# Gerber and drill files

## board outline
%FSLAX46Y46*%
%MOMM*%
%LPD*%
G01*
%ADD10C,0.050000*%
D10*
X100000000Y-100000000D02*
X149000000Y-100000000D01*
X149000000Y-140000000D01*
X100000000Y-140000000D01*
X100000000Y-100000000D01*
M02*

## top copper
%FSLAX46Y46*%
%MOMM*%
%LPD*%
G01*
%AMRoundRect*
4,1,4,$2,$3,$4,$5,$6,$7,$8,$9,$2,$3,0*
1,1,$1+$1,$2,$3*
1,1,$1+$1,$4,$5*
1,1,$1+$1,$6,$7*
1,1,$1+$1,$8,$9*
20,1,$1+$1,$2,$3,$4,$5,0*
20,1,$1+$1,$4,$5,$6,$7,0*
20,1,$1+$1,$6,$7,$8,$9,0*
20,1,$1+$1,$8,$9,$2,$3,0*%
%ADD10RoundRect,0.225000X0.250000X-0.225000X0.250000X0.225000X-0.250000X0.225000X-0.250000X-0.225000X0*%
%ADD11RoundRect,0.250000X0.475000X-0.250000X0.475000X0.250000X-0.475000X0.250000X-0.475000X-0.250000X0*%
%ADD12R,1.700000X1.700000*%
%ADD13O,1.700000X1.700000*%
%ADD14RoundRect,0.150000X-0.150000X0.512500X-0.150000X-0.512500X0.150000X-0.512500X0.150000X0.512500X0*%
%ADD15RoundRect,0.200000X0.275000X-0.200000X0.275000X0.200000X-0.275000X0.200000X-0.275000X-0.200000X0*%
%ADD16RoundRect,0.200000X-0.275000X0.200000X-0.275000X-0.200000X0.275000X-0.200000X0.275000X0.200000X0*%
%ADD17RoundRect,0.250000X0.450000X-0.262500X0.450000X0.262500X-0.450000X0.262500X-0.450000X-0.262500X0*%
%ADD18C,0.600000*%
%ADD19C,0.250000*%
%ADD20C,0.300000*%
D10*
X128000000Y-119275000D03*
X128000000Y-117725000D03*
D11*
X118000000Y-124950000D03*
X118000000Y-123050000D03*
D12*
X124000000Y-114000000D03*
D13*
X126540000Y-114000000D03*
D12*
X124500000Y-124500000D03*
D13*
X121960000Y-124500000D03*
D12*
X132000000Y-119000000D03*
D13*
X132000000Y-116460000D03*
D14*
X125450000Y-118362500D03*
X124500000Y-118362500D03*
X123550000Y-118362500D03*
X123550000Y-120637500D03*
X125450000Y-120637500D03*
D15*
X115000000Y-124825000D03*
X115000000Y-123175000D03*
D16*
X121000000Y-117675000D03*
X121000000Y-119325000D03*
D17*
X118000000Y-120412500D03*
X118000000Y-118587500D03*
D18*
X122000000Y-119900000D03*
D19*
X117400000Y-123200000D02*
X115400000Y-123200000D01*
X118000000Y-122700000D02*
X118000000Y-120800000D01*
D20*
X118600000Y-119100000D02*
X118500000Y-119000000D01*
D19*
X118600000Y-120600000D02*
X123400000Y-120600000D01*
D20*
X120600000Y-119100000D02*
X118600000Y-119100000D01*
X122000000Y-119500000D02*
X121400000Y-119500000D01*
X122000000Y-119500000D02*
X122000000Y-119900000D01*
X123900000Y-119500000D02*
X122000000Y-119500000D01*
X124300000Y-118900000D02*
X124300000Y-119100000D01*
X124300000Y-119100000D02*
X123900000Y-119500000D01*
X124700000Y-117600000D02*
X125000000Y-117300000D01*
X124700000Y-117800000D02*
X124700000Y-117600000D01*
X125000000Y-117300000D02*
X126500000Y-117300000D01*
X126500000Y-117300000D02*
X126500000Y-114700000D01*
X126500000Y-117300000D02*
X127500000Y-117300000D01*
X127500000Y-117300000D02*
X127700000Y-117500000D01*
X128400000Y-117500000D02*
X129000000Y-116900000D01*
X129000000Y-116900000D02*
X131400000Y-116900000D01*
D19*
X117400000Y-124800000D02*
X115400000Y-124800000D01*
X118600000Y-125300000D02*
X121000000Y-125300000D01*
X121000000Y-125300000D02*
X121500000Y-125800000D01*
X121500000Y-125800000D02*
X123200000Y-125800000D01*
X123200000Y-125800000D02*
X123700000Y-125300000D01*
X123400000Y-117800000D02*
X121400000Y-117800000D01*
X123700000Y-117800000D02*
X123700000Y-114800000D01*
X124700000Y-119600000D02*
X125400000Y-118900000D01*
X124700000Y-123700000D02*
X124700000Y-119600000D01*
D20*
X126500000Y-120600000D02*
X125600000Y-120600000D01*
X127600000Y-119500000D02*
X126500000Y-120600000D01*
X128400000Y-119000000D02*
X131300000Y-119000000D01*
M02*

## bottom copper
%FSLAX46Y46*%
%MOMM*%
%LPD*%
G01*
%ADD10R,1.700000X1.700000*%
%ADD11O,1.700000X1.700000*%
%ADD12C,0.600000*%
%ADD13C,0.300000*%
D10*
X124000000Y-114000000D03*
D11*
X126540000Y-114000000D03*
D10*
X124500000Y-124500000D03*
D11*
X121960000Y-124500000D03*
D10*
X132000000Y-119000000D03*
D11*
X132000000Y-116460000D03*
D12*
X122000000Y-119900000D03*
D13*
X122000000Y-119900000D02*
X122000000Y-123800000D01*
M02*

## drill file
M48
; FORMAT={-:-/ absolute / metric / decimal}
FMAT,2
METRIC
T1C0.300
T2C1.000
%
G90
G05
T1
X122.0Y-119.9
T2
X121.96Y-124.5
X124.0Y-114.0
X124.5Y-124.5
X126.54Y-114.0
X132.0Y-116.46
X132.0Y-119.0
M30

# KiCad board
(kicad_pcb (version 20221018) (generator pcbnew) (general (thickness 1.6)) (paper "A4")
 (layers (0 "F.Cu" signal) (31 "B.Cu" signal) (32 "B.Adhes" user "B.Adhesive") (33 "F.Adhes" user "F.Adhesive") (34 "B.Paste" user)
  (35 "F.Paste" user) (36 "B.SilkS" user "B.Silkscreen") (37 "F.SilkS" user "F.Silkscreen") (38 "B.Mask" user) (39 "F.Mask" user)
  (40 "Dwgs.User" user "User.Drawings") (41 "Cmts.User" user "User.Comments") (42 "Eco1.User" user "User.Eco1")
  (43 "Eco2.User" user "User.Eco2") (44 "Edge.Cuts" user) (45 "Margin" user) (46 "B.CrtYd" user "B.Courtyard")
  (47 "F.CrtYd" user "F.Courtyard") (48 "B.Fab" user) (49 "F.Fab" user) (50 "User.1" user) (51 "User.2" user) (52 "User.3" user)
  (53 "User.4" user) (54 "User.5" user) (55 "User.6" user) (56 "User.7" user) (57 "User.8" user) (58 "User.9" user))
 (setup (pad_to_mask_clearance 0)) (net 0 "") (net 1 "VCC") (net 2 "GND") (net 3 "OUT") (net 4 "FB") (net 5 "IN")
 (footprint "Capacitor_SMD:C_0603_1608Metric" (layer "F.Cu") (at 128 118.5 90)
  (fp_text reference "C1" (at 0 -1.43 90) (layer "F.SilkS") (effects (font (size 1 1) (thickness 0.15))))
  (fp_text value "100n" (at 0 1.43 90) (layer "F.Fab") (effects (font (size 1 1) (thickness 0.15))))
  (pad "1" smd roundrect (at -0.775 0 90) (size 0.9 0.95) (layers "F.Cu" "F.Paste" "F.Mask") (roundrect_rratio 0.25) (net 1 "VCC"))
  (pad "2" smd roundrect (at 0.775 0 90) (size 0.9 0.95) (layers "F.Cu" "F.Paste" "F.Mask") (roundrect_rratio 0.25) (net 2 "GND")))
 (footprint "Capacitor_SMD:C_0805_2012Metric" (layer "F.Cu") (at 118 124 90)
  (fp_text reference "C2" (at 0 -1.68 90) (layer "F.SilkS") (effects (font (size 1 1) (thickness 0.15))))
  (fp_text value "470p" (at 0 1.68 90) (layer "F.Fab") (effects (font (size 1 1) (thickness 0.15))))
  (pad "1" smd roundrect (at -0.95 0 90) (size 1 1.45) (layers "F.Cu" "F.Paste" "F.Mask") (roundrect_rratio 0.25) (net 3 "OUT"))
  (pad "2" smd roundrect (at 0.95 0 90) (size 1 1.45) (layers "F.Cu" "F.Paste" "F.Mask") (roundrect_rratio 0.25) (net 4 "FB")))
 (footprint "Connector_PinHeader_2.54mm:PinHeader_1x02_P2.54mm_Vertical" (layer "F.Cu") (at 124 114 90)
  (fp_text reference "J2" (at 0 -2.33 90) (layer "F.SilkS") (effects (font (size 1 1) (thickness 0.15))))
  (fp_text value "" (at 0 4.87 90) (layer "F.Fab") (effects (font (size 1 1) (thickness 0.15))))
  (pad "1" thru_hole rect (at 0 0 90) (size 1.7 1.7) (drill 1) (layers "*.Cu" "*.Mask") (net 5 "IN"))
  (pad "2" thru_hole oval (at 0 2.54 90) (size 1.7 1.7) (drill 1) (layers "*.Cu" "*.Mask") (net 2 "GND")))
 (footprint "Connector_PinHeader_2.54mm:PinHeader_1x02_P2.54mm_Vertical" (layer "F.Cu") (at 124.5 124.5 -90)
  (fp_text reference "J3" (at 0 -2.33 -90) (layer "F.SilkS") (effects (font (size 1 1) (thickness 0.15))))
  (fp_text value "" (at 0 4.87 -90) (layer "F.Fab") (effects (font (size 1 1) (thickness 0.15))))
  (pad "1" thru_hole rect (at 0 0 270) (size 1.7 1.7) (drill 1) (layers "*.Cu" "*.Mask") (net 3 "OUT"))
  (pad "2" thru_hole oval (at 0 2.54 270) (size 1.7 1.7) (drill 1) (layers "*.Cu" "*.Mask") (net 2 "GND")))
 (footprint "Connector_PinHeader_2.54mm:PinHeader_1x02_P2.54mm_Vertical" (layer "F.Cu") (at 132 119 180)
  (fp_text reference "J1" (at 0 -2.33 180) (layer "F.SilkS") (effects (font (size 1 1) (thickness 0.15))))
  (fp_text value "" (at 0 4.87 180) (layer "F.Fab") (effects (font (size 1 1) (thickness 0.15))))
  (pad "1" thru_hole rect (at 0 0 180) (size 1.7 1.7) (drill 1) (layers "*.Cu" "*.Mask") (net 1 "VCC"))
  (pad "2" thru_hole oval (at 0 2.54 180) (size 1.7 1.7) (drill 1) (layers "*.Cu" "*.Mask") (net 2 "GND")))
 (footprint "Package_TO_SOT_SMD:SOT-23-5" (layer "F.Cu") (at 124.5 119.5 -90)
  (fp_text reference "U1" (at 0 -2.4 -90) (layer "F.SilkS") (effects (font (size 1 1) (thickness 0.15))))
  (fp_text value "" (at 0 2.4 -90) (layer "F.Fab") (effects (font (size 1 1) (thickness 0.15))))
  (pad "1" smd roundrect (at -1.1375 -0.95 270) (size 1.325 0.6) (layers "F.Cu" "F.Paste" "F.Mask") (roundrect_rratio 0.25) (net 3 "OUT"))
  (pad "2" smd roundrect (at -1.1375 0 270) (size 1.325 0.6) (layers "F.Cu" "F.Paste" "F.Mask") (roundrect_rratio 0.25) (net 2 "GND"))
  (pad "3" smd roundrect (at -1.1375 0.95 270) (size 1.325 0.6) (layers "F.Cu" "F.Paste" "F.Mask") (roundrect_rratio 0.25) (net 5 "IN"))
  (pad "4" smd roundrect (at 1.1375 0.95 270) (size 1.325 0.6) (layers "F.Cu" "F.Paste" "F.Mask") (roundrect_rratio 0.25) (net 4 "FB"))
  (pad "5" smd roundrect (at 1.1375 -0.95 270) (size 1.325 0.6) (layers "F.Cu" "F.Paste" "F.Mask") (roundrect_rratio 0.25) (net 1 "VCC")))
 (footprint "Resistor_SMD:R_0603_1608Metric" (layer "F.Cu") (at 115 124 90)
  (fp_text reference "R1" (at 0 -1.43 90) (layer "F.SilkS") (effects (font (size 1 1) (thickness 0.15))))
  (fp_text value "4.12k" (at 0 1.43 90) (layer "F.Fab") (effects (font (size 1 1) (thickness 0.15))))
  (pad "1" smd roundrect (at -0.825 0 90) (size 0.8 0.95) (layers "F.Cu" "F.Paste" "F.Mask") (roundrect_rratio 0.25) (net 3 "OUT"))
  (pad "2" smd roundrect (at 0.825 0 90) (size 0.8 0.95) (layers "F.Cu" "F.Paste" "F.Mask") (roundrect_rratio 0.25) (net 4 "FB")))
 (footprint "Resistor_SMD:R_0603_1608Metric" (layer "F.Cu") (at 121 118.5 -90)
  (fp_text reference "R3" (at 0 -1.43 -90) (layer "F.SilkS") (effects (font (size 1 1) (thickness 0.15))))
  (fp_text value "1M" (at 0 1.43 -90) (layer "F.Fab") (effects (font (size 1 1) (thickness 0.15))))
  (pad "1" smd roundrect (at -0.825 0 270) (size 0.8 0.95) (layers "F.Cu" "F.Paste" "F.Mask") (roundrect_rratio 0.25) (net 5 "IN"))
  (pad "2" smd roundrect (at 0.825 0 270) (size 0.8 0.95) (layers "F.Cu" "F.Paste" "F.Mask") (roundrect_rratio 0.25) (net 2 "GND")))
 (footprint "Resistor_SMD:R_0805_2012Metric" (layer "F.Cu") (at 118 119.5 90)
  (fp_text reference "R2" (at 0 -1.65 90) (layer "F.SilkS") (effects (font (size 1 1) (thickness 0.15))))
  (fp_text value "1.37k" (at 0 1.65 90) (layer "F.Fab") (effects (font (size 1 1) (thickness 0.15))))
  (pad "1" smd roundrect (at -0.9125 0 90) (size 1.025 1.4) (layers "F.Cu" "F.Paste" "F.Mask") (roundrect_rratio 0.243902) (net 4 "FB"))
  (pad "2" smd roundrect (at 0.9125 0 90) (size 1.025 1.4) (layers "F.Cu" "F.Paste" "F.Mask") (roundrect_rratio 0.243902) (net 2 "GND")))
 (gr_rect (start 100 100) (end 149 140) (stroke (width 0.05) (type default)) (fill none) (layer "Edge.Cuts"))
 (segment (start 117.4 123.2) (end 115.4 123.2) (width 0.25) (layer "F.Cu") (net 4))
 (segment (start 118 122.7) (end 118 120.8) (width 0.25) (layer "F.Cu") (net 4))
 (segment (start 118.6 119.1) (end 118.5 119) (width 0.3) (layer "F.Cu") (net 2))
 (segment (start 118.6 120.6) (end 123.4 120.6) (width 0.25) (layer "F.Cu") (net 4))
 (segment (start 120.6 119.1) (end 118.6 119.1) (width 0.3) (layer "F.Cu") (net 2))
 (segment (start 122 119.5) (end 121.4 119.5) (width 0.3) (layer "F.Cu") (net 2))
 (segment (start 122 119.5) (end 122 119.9) (width 0.3) (layer "F.Cu") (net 2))
 (segment (start 123.9 119.5) (end 122 119.5) (width 0.3) (layer "F.Cu") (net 2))
 (segment (start 124.3 118.9) (end 124.3 119.1) (width 0.3) (layer "F.Cu") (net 2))
 (segment (start 124.3 119.1) (end 123.9 119.5) (width 0.3) (layer "F.Cu") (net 2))
 (segment (start 124.7 117.6) (end 125 117.3) (width 0.3) (layer "F.Cu") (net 2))
 (segment (start 124.7 117.8) (end 124.7 117.6) (width 0.3) (layer "F.Cu") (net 2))
 (segment (start 125 117.3) (end 126.5 117.3) (width 0.3) (layer "F.Cu") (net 2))
 (segment (start 126.5 117.3) (end 126.5 114.7) (width 0.3) (layer "F.Cu") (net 2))
 (segment (start 126.5 117.3) (end 127.5 117.3) (width 0.3) (layer "F.Cu") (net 2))
 (segment (start 127.5 117.3) (end 127.7 117.5) (width 0.3) (layer "F.Cu") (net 2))
 (segment (start 128.4 117.5) (end 129 116.9) (width 0.3) (layer "F.Cu") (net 2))
 (segment (start 129 116.9) (end 131.4 116.9) (width 0.3) (layer "F.Cu") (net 2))
 (via (at 122 119.9) (size 0.6) (drill 0.3) (layers "F.Cu" "B.Cu") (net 2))
 (segment (start 117.4 124.8) (end 115.4 124.8) (width 0.25) (layer "F.Cu") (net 3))
 (segment (start 118.6 125.3) (end 121 125.3) (width 0.25) (layer "F.Cu") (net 3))
 (segment (start 121 125.3) (end 121.5 125.8) (width 0.25) (layer "F.Cu") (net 3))
 (segment (start 121.5 125.8) (end 123.2 125.8) (width 0.25) (layer "F.Cu") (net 3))
 (segment (start 122 119.9) (end 122 123.8) (width 0.3) (layer "B.Cu") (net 2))
 (segment (start 123.2 125.8) (end 123.7 125.3) (width 0.25) (layer "F.Cu") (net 3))
 (segment (start 123.4 117.8) (end 121.4 117.8) (width 0.25) (layer "F.Cu") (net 5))
 (segment (start 123.7 117.8) (end 123.7 114.8) (width 0.25) (layer "F.Cu") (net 5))
 (segment (start 124.7 119.6) (end 125.4 118.9) (width 0.25) (layer "F.Cu") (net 3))
 (segment (start 124.7 123.7) (end 124.7 119.6) (width 0.25) (layer "F.Cu") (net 3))
 (segment (start 126.5 120.6) (end 125.6 120.6) (width 0.3) (layer "F.Cu") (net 1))
 (segment (start 127.6 119.5) (end 126.5 120.6) (width 0.3) (layer "F.Cu") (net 1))
 (segment (start 128.4 119) (end 131.3 119) (width 0.3) (layer "F.Cu") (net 1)))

